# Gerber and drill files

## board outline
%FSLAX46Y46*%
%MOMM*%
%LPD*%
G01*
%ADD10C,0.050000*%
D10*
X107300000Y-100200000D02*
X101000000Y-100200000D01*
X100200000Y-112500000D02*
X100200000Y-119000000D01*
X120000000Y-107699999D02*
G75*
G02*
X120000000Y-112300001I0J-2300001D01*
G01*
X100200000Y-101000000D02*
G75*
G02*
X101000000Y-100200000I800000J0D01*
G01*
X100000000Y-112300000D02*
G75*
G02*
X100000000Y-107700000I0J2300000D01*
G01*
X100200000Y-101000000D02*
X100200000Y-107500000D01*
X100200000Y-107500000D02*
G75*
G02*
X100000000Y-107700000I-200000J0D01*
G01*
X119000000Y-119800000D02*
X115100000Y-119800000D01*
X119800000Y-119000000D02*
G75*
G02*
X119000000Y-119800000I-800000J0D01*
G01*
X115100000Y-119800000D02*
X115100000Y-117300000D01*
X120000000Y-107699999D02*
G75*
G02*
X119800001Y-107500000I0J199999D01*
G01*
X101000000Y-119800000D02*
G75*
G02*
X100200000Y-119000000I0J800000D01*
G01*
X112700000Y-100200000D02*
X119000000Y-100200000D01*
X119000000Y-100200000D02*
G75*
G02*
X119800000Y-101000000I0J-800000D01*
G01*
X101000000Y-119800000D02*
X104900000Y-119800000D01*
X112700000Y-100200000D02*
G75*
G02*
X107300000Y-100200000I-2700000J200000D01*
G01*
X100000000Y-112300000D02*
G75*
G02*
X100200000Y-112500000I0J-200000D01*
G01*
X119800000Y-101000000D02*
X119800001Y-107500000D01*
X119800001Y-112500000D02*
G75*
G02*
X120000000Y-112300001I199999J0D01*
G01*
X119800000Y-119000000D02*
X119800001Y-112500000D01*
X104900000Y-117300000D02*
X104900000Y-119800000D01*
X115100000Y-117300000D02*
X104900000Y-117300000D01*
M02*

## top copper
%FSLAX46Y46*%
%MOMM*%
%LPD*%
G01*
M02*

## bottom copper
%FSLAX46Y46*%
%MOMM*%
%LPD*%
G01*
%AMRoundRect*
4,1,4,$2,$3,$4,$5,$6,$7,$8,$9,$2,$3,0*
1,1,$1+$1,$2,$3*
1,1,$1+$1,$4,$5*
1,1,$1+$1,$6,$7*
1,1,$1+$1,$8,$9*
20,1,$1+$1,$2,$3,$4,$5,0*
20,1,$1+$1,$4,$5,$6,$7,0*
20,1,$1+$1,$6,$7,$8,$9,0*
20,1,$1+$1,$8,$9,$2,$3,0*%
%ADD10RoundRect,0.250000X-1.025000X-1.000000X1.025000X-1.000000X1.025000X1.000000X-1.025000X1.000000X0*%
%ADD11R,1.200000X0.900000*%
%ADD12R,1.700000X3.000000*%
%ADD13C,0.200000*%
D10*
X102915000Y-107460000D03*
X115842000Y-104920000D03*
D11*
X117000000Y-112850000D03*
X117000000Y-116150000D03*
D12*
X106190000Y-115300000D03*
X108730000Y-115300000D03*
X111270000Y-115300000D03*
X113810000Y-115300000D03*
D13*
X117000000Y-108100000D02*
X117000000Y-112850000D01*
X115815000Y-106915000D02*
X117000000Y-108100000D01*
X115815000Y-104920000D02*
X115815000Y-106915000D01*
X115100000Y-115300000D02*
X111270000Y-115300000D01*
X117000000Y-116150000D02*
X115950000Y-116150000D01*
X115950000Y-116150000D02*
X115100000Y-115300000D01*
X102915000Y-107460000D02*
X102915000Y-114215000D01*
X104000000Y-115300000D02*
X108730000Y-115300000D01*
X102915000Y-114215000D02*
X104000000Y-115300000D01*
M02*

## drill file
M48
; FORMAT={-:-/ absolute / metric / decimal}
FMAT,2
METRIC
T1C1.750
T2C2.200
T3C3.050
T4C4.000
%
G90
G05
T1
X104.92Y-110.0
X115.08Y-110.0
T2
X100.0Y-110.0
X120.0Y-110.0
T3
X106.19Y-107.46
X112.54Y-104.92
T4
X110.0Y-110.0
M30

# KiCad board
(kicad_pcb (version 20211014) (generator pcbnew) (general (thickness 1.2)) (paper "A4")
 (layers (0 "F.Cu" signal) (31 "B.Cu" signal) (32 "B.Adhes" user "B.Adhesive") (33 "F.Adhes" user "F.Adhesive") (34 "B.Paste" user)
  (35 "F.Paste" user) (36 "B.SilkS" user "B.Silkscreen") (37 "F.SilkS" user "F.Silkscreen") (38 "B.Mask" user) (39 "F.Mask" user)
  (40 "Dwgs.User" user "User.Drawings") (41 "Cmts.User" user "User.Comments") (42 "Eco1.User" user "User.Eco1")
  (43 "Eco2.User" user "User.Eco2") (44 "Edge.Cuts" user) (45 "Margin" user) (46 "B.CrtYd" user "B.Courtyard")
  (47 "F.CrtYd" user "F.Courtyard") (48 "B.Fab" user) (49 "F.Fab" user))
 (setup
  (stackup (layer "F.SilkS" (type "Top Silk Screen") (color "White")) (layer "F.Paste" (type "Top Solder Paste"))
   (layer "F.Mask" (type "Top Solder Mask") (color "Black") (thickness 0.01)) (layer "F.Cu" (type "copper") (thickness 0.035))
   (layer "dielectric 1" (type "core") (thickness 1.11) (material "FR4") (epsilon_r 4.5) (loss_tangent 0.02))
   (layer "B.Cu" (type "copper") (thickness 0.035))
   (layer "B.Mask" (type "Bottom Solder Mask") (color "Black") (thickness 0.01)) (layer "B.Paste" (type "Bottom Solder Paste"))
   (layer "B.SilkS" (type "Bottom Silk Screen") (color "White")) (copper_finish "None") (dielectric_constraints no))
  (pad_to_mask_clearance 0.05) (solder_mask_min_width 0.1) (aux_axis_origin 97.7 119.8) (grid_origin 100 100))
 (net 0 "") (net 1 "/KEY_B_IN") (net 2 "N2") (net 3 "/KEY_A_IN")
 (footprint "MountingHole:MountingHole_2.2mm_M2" (layer "F.Cu") (at 120 110)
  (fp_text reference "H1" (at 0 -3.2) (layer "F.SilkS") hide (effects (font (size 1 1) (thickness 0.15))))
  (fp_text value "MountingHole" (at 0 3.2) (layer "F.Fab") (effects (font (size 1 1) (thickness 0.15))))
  (pad "" np_thru_hole circle (at 0 0) (size 2.2 2.2) (drill 2.2) (layers *.Cu *.Mask)))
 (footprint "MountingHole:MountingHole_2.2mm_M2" (layer "F.Cu") (at 100 110)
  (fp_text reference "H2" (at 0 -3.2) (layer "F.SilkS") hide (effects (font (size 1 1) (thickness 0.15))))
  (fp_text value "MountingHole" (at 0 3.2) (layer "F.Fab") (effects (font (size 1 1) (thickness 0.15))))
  (pad "" np_thru_hole circle (at 0 0) (size 2.2 2.2) (drill 2.2) (layers *.Cu *.Mask)))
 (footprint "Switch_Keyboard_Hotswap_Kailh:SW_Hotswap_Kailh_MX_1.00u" (layer "F.Cu") (at 110 110)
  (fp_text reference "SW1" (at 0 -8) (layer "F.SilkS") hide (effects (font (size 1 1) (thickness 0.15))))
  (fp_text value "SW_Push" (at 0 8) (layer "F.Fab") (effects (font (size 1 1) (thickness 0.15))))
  (pad "" np_thru_hole circle locked (at 5.08 0) (size 1.75 1.75) (drill 1.75) (layers *.Cu *.Mask))
  (pad "" np_thru_hole circle locked (at 2.54 -5.08) (size 3.05 3.05) (drill 3.05) (layers *.Cu *.Mask))
  (pad "" np_thru_hole circle locked (at -3.81 -2.54) (size 3.05 3.05) (drill 3.05) (layers *.Cu *.Mask))
  (pad "" np_thru_hole circle locked (at -5.08 0) (size 1.75 1.75) (drill 1.75) (layers *.Cu *.Mask))
  (pad "" np_thru_hole circle locked (at 0 0) (size 4 4) (drill 4) (layers *.Cu *.Mask))
  (pad "1" smd roundrect locked (at -7.085 -2.54) (size 2.55 2.5) (layers "B.Cu" "B.Paste" "B.Mask") (roundrect_rratio 0.1)
   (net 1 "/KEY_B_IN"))
  (pad "2" smd roundrect locked (at 5.842 -5.08) (size 2.55 2.5) (layers "B.Cu" "B.Paste" "B.Mask") (roundrect_rratio 0.1) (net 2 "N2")))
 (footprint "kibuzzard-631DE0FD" (layer "F.Cu") (at 113.81 114.92 90)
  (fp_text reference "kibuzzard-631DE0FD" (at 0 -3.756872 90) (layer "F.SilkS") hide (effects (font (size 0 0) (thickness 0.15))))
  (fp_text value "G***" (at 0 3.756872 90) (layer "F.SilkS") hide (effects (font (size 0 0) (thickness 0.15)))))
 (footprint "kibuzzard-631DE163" (layer "F.Cu") (at 103.5 101.5)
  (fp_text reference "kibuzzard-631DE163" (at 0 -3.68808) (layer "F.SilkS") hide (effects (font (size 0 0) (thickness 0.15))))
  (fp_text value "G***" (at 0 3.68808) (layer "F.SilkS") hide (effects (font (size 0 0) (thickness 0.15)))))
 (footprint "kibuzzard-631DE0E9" (layer "F.Cu") (at 111.27 114.92 90)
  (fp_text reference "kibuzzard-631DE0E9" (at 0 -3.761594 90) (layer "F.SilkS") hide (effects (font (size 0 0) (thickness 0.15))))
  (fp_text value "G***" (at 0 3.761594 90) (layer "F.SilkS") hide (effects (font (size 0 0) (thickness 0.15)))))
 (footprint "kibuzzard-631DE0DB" (layer "F.Cu") (at 108.73 114.92 90)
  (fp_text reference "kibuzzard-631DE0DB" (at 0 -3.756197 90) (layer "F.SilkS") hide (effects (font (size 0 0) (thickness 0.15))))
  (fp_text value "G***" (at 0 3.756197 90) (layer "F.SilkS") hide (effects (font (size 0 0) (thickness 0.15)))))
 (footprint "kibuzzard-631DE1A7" (layer "F.Cu") (at 102.5 118.5)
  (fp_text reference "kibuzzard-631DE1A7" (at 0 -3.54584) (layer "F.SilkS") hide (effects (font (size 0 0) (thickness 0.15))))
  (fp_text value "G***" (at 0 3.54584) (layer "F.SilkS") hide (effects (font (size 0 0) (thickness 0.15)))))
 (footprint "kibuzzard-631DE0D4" (layer "F.Cu") (at 106.19 114.92 90)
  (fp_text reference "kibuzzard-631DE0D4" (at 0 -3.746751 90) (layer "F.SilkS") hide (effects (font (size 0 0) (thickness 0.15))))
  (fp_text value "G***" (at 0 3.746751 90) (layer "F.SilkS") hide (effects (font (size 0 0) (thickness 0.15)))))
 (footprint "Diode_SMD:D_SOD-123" (layer "B.Cu") (at 117 114.5 -90)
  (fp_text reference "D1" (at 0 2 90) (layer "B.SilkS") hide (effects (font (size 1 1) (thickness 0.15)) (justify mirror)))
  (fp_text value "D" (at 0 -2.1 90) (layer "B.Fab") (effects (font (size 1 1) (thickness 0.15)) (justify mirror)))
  (pad "1" smd rect (at -1.65 0 270) (size 0.9 1.2) (layers "B.Cu" "B.Paste" "B.Mask") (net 2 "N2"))
  (pad "2" smd rect (at 1.65 0 270) (size 0.9 1.2) (layers "B.Cu" "B.Paste" "B.Mask") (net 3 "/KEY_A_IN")))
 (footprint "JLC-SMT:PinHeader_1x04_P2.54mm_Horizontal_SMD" (layer "B.Cu") (at 106.19 117.3 -90)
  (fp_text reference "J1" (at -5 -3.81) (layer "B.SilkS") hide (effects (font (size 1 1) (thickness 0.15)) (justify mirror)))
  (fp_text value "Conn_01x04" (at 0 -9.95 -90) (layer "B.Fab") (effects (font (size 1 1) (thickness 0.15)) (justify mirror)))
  (pad "1" smd rect (at -2 0 270) (size 3 1.7) (layers "B.Cu" "B.Paste" "B.Mask") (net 1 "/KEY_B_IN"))
  (pad "2" smd rect (at -2 -2.54 270) (size 3 1.7) (layers "B.Cu" "B.Paste" "B.Mask") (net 1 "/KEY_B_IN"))
  (pad "3" smd rect (at -2 -5.08 270) (size 3 1.7) (layers "B.Cu" "B.Paste" "B.Mask") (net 3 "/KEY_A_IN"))
  (pad "4" smd rect (at -2 -7.62 270) (size 3 1.7) (layers "B.Cu" "B.Paste" "B.Mask") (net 3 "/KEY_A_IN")))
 (gr_line (start 107.3 100.2) (end 101 100.2) (layer "Edge.Cuts") (width 0.05))
 (gr_line (start 100.2 112.5) (end 100.2 119) (layer "Edge.Cuts") (width 0.05))
 (gr_arc (start 120 107.699999) (mid 122.300001 110) (end 120 112.300001) (layer "Edge.Cuts") (width 0.05))
 (gr_arc (start 100.2 101) (mid 100.434315 100.434315) (end 101 100.2) (layer "Edge.Cuts") (width 0.05))
 (gr_arc (start 100 112.3) (mid 97.7 110) (end 100 107.7) (layer "Edge.Cuts") (width 0.05))
 (gr_line (start 100.2 101) (end 100.2 107.5) (layer "Edge.Cuts") (width 0.05))
 (gr_arc (start 100.2 107.5) (mid 100.141421 107.641421) (end 100 107.7) (layer "Edge.Cuts") (width 0.05))
 (gr_line (start 119 119.8) (end 115.1 119.8) (layer "Edge.Cuts") (width 0.05))
 (gr_arc (start 119.8 119) (mid 119.565685 119.565685) (end 119 119.8) (layer "Edge.Cuts") (width 0.05))
 (gr_line (start 115.1 119.8) (end 115.1 117.3) (layer "Edge.Cuts") (width 0.05))
 (gr_arc (start 120 107.699999) (mid 119.858579 107.641421) (end 119.800001 107.5) (layer "Edge.Cuts") (width 0.05))
 (gr_arc (start 101 119.8) (mid 100.434315 119.565685) (end 100.2 119) (layer "Edge.Cuts") (width 0.05))
 (gr_line (start 112.7 100.2) (end 119 100.2) (layer "Edge.Cuts") (width 0.05))
 (gr_arc (start 119 100.2) (mid 119.565685 100.434315) (end 119.8 101) (layer "Edge.Cuts") (width 0.05))
 (gr_line (start 101 119.8) (end 104.9 119.8) (layer "Edge.Cuts") (width 0.05))
 (gr_arc (start 112.7 100.2) (mid 110 102.707397) (end 107.3 100.2) (layer "Edge.Cuts") (width 0.05))
 (gr_arc (start 100 112.3) (mid 100.141421 112.358579) (end 100.2 112.5) (layer "Edge.Cuts") (width 0.05))
 (gr_line (start 119.8 101) (end 119.800001 107.5) (layer "Edge.Cuts") (width 0.05))
 (gr_arc (start 119.800001 112.5) (mid 119.858579 112.358579) (end 120 112.300001) (layer "Edge.Cuts") (width 0.05))
 (gr_line (start 119.8 119) (end 119.800001 112.5) (layer "Edge.Cuts") (width 0.05))
 (gr_line (start 104.9 117.3) (end 104.9 119.8) (layer "Edge.Cuts") (width 0.05))
 (gr_line (start 115.1 117.3) (end 104.9 117.3) (layer "Edge.Cuts") (width 0.05))
 (segment (start 117 108.1) (end 117 112.85) (width 0.2) (layer "B.Cu") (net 2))
 (segment (start 115.815 106.915) (end 117 108.1) (width 0.2) (layer "B.Cu") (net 2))
 (segment (start 115.815 104.92) (end 115.815 106.915) (width 0.2) (layer "B.Cu") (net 2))
 (segment (start 115.1 115.3) (end 111.27 115.3) (width 0.2) (layer "B.Cu") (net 3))
 (segment (start 117 116.15) (end 115.95 116.15) (width 0.2) (layer "B.Cu") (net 3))
 (segment (start 115.95 116.15) (end 115.1 115.3) (width 0.2) (layer "B.Cu") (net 3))
 (segment (start 102.915 107.46) (end 102.915 114.215) (width 0.2) (layer "B.Cu") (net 1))
 (segment (start 104 115.3) (end 108.73 115.3) (width 0.2) (layer "B.Cu") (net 1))
 (segment (start 102.915 114.215) (end 104 115.3) (width 0.2) (layer "B.Cu") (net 1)))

